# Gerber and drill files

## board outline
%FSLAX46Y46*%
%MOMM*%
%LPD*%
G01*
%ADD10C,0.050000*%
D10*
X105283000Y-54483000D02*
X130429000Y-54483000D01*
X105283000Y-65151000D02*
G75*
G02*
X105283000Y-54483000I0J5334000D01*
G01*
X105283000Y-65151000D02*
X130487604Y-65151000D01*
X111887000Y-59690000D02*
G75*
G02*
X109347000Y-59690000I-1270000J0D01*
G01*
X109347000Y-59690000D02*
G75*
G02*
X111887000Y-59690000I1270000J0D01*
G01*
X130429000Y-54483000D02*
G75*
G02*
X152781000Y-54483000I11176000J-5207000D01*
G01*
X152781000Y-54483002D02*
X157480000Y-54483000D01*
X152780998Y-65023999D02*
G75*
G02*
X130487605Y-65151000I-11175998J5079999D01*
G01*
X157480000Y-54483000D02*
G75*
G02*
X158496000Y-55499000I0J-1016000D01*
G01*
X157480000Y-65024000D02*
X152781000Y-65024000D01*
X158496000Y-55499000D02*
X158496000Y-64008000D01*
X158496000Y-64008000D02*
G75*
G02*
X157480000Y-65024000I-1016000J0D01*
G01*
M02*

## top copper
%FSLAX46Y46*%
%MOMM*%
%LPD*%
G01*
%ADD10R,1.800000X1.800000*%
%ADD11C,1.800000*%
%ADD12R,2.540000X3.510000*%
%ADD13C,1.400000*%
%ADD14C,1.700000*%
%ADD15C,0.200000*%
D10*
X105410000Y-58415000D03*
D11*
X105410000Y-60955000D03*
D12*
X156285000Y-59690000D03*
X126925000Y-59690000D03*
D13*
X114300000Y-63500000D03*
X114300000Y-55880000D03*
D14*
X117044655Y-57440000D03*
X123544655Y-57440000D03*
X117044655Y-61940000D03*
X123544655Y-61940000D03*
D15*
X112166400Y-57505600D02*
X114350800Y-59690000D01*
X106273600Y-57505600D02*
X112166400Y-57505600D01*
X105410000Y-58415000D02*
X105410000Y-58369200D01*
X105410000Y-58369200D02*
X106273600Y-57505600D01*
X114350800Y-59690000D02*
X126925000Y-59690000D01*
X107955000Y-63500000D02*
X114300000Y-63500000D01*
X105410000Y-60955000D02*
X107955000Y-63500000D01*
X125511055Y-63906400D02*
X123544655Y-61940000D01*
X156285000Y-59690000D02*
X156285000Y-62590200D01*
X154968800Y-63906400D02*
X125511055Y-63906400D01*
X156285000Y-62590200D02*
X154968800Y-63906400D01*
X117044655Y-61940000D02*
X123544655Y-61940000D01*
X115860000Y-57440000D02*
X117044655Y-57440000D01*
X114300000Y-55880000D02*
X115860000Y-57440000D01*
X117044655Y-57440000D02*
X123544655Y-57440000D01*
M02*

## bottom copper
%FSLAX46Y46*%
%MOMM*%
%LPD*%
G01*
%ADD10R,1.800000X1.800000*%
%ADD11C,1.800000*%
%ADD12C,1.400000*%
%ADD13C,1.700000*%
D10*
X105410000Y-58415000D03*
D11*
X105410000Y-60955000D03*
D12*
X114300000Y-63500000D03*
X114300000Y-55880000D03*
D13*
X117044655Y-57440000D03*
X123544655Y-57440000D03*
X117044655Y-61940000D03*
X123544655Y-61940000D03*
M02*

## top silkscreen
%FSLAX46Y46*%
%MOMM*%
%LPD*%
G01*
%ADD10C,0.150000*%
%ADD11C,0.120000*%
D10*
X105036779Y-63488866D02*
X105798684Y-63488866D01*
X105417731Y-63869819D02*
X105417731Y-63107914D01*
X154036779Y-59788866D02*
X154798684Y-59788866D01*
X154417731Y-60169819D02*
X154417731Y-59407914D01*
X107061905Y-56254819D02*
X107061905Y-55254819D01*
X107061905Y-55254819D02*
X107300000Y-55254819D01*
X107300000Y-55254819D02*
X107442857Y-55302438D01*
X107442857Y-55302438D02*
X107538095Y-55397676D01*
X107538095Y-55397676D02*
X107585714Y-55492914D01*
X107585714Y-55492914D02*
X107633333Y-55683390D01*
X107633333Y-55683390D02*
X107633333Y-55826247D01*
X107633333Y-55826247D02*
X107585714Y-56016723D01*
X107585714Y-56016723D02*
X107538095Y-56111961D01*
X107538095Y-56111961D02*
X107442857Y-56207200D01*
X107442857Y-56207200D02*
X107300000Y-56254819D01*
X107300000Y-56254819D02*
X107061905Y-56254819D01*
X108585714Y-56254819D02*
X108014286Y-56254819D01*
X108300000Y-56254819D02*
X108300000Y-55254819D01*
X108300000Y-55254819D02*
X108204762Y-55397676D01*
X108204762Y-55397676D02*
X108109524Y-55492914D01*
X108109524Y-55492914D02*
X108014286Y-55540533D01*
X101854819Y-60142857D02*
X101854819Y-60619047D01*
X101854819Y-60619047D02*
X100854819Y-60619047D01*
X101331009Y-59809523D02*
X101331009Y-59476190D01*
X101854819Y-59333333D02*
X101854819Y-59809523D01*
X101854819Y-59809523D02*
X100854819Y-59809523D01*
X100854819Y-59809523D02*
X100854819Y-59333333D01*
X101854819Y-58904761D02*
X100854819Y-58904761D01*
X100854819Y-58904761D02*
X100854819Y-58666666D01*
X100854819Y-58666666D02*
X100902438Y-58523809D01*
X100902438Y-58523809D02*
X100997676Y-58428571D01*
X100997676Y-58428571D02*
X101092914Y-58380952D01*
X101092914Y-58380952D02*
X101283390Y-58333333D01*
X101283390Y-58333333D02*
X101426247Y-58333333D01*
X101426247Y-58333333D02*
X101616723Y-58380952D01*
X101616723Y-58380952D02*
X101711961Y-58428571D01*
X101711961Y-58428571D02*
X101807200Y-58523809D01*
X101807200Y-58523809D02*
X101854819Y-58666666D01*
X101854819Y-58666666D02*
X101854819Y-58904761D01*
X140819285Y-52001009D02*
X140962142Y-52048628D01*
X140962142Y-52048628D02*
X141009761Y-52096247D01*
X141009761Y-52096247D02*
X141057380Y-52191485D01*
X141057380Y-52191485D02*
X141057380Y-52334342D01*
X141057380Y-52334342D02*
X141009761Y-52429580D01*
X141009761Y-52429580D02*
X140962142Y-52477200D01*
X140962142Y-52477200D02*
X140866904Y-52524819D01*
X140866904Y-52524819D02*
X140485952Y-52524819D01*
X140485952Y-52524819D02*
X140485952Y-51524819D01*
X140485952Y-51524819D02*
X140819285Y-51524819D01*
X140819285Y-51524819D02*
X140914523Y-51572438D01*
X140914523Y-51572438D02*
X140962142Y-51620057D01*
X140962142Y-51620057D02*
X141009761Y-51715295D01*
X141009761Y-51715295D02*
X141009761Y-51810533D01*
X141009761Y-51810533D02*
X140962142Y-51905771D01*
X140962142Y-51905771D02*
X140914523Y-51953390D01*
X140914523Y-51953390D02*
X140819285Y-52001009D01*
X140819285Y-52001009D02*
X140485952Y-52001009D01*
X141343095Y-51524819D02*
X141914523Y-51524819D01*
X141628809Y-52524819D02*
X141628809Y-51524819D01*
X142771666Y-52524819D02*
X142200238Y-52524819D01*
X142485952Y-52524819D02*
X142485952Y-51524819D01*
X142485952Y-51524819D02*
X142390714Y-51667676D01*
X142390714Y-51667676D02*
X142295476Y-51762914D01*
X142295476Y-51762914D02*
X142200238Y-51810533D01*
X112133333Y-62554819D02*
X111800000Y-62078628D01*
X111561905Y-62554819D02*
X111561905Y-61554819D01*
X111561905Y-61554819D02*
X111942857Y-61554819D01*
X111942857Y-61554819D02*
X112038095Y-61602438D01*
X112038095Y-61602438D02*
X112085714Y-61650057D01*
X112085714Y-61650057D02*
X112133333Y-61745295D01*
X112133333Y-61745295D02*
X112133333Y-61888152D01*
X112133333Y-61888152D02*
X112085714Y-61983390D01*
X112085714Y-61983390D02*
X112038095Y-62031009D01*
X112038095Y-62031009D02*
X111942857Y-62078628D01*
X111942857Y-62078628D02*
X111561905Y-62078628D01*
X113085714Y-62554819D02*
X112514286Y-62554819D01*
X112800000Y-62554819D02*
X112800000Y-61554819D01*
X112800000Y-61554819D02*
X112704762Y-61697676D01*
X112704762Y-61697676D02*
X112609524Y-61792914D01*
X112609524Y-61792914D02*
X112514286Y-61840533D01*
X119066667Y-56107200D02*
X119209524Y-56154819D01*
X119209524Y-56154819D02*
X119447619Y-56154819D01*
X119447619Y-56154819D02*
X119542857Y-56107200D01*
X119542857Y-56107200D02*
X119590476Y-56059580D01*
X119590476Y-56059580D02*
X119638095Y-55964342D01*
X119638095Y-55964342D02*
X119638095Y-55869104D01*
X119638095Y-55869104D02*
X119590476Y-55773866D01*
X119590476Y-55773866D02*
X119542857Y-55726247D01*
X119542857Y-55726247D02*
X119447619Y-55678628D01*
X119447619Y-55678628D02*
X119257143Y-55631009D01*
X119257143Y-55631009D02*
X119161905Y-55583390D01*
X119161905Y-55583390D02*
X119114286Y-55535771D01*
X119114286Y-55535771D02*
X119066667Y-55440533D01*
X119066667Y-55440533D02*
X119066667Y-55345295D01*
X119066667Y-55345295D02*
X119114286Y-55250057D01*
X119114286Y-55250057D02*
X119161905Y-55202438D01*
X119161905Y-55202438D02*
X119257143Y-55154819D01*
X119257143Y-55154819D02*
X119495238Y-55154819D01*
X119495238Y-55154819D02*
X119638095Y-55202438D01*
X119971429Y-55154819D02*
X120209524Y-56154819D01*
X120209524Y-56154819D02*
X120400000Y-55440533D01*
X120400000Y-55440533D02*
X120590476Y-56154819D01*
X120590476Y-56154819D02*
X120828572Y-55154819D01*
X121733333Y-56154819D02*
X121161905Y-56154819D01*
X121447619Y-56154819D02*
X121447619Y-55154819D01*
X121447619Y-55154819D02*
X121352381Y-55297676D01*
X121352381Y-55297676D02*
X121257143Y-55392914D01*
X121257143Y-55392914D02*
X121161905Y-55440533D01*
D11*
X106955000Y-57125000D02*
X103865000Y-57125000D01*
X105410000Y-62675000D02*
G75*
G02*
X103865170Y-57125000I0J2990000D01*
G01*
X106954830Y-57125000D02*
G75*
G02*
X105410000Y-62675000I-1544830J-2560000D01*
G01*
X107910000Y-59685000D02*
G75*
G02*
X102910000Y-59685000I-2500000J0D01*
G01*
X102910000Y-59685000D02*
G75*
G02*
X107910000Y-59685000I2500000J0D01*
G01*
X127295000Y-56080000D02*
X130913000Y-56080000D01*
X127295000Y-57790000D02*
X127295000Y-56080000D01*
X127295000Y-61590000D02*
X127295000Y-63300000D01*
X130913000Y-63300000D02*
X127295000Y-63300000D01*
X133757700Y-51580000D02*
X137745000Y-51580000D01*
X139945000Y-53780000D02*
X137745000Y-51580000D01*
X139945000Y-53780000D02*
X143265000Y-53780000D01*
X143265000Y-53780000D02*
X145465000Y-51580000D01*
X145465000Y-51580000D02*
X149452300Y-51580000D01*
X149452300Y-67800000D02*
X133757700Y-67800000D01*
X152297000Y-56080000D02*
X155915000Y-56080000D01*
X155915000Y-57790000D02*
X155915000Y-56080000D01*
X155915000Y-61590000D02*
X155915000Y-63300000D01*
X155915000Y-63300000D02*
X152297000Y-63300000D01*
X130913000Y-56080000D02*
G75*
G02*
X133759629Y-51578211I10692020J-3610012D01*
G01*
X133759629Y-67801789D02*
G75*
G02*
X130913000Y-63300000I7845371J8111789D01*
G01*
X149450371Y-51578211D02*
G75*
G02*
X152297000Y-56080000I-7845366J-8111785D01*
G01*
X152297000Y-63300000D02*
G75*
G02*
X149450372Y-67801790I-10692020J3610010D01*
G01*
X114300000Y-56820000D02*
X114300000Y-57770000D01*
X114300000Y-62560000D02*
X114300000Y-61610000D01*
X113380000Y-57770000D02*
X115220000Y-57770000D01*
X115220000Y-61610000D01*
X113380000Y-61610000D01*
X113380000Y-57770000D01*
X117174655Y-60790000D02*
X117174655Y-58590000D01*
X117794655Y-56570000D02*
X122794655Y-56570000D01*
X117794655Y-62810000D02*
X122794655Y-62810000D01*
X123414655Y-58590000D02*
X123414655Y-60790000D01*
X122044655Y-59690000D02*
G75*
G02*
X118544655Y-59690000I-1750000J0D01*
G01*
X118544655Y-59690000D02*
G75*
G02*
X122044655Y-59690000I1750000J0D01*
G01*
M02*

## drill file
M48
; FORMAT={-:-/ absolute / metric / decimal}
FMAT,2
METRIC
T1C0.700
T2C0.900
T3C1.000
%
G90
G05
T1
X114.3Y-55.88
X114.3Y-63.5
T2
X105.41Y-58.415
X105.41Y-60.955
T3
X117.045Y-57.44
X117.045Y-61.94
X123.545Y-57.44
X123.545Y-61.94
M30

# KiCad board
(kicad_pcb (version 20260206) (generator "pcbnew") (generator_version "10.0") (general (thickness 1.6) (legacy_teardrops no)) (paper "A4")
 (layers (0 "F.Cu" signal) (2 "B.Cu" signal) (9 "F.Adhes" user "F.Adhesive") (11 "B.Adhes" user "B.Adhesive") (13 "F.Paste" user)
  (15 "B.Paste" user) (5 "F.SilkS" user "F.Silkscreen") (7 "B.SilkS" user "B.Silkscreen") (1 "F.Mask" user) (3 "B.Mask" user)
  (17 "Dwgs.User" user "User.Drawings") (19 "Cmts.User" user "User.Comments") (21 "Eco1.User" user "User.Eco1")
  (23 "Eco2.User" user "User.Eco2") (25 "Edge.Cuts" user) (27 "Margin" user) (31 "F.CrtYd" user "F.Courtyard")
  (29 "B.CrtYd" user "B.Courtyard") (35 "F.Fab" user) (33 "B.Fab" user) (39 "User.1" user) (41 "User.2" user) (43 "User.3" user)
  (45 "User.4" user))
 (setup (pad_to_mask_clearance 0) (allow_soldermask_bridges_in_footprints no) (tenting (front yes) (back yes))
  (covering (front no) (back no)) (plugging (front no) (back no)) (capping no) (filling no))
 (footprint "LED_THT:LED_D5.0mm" (layer "F.Cu") (at 105.41 58.415 -90)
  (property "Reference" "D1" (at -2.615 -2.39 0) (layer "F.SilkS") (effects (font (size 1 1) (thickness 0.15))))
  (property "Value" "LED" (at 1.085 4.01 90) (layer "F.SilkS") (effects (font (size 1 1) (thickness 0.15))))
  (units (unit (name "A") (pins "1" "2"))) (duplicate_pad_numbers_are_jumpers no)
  (fp_line (start -1.29 -1.545) (end -1.29 1.545) (stroke (width 0.12) (type solid)) (layer "F.SilkS"))
  (fp_arc (start 4.26 0) (mid 2.071779 2.880495) (end -1.29 1.54483) (stroke (width 0.12) (type solid)) (layer "F.SilkS"))
  (fp_arc (start -1.29 -1.54483) (mid 2.071779 -2.880495) (end 4.26 0) (stroke (width 0.12) (type solid)) (layer "F.SilkS"))
  (fp_circle (center 1.27 0) (end 3.77 0) (stroke (width 0.12) (type solid)) (fill no) (layer "F.SilkS"))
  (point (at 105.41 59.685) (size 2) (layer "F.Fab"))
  (pad "1" thru_hole rect (at 0 0 270) (size 1.8 1.8) (drill 0.9) (layers "*.Cu" "*.Mask") (remove_unused_layers no) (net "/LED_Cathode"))
  (pad "2" thru_hole circle (at 2.54 0 270) (size 1.8 1.8) (drill 0.9) (layers "*.Cu" "*.Mask") (remove_unused_layers no) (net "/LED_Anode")))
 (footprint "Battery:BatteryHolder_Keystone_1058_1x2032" (layer "F.Cu") (at 141.605 59.69 180)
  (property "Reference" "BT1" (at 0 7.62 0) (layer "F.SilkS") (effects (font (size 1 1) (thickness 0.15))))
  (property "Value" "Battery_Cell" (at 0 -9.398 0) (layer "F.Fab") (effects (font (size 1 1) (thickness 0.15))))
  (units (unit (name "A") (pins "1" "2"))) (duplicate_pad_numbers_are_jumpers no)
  (fp_line (start 14.31 3.61) (end 10.692 3.61) (stroke (width 0.12) (type solid)) (layer "F.SilkS"))
  (fp_line (start 14.31 1.9) (end 14.31 3.61) (stroke (width 0.12) (type solid)) (layer "F.SilkS"))
  (fp_line (start 14.31 -1.9) (end 14.31 -3.61) (stroke (width 0.12) (type solid)) (layer "F.SilkS"))
  (fp_line (start 10.692 -3.61) (end 14.31 -3.61) (stroke (width 0.12) (type solid)) (layer "F.SilkS"))
  (fp_line (start 7.8473 8.11) (end 3.86 8.11) (stroke (width 0.12) (type solid)) (layer "F.SilkS"))
  (fp_line (start 1.66 5.91) (end 3.86 8.11) (stroke (width 0.12) (type solid)) (layer "F.SilkS"))
  (fp_line (start 1.66 5.91) (end -1.66 5.91) (stroke (width 0.12) (type solid)) (layer "F.SilkS"))
  (fp_line (start -1.66 5.91) (end -3.86 8.11) (stroke (width 0.12) (type solid)) (layer "F.SilkS"))
  (fp_line (start -3.86 8.11) (end -7.8473 8.11) (stroke (width 0.12) (type solid)) (layer "F.SilkS"))
  (fp_line (start -7.8473 -8.11) (end 7.8473 -8.11) (stroke (width 0.12) (type solid)) (layer "F.SilkS"))
  (fp_line (start -10.692 3.61) (end -14.31 3.61) (stroke (width 0.12) (type solid)) (layer "F.SilkS"))
  (fp_line (start -14.31 1.9) (end -14.31 3.61) (stroke (width 0.12) (type solid)) (layer "F.SilkS"))
  (fp_line (start -14.31 -1.9) (end -14.31 -3.61) (stroke (width 0.12) (type solid)) (layer "F.SilkS"))
  (fp_line (start -14.31 -3.61) (end -10.692 -3.61) (stroke (width 0.12) (type solid)) (layer "F.SilkS"))
  (fp_arc (start 10.692 3.61) (mid 9.538084 6.031244) (end 7.845371 8.111789) (stroke (width 0.12) (type solid)) (layer "F.SilkS"))
  (fp_arc (start 7.845371 -8.111789) (mid 9.538085 -6.031244) (end 10.692 -3.61) (stroke (width 0.12) (type solid)) (layer "F.SilkS"))
  (fp_arc (start -7.845371 8.111789) (mid -9.538085 6.031244) (end -10.692 3.61) (stroke (width 0.12) (type solid)) (layer "F.SilkS"))
  (fp_arc (start -10.692 -3.61) (mid -9.538084 -6.031244) (end -7.845371 -8.111789) (stroke (width 0.12) (type solid)) (layer "F.SilkS"))
  (pad "1" smd rect (at -14.68 0 180) (size 2.54 3.51) (layers "F.Cu" "F.Mask" "F.Paste") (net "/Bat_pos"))
  (pad "2" smd rect (at 14.68 0 180) (size 2.54 3.51) (layers "F.Cu" "F.Mask" "F.Paste") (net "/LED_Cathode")))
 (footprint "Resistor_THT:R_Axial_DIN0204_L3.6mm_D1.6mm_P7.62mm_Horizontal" (layer "F.Cu") (at 114.3 63.5 90)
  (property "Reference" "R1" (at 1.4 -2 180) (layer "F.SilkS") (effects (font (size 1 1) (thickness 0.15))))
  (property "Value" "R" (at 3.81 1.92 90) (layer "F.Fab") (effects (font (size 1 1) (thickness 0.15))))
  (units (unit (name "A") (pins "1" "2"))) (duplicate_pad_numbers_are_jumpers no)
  (fp_line (start 6.68 0) (end 5.73 0) (stroke (width 0.12) (type solid)) (layer "F.SilkS"))
  (fp_line (start 0.94 0) (end 1.89 0) (stroke (width 0.12) (type solid)) (layer "F.SilkS"))
  (fp_rect (start 1.89 -0.92) (end 5.73 0.92) (stroke (width 0.12) (type solid)) (fill no) (layer "F.SilkS"))
  (pad "1" thru_hole circle (at 0 0 90) (size 1.4 1.4) (drill 0.7) (layers "*.Cu" "*.Mask") (remove_unused_layers no) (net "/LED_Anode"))
  (pad "2" thru_hole circle (at 7.62 0 90) (size 1.4 1.4) (drill 0.7) (layers "*.Cu" "*.Mask") (remove_unused_layers no)
   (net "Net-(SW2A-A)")))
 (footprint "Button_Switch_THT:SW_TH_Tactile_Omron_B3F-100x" (layer "F.Cu") (at 117.044655 57.44)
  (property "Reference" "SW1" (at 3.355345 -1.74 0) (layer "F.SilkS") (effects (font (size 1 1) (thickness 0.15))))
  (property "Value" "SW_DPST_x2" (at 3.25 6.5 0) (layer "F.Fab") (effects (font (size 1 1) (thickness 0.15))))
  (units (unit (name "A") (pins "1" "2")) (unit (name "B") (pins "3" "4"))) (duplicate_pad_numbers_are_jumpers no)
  (fp_line (start 0.13 3.35) (end 0.13 1.15) (stroke (width 0.12) (type solid)) (layer "F.SilkS"))
  (fp_line (start 0.75 -0.87) (end 5.75 -0.87) (stroke (width 0.12) (type solid)) (layer "F.SilkS"))
  (fp_line (start 0.75 5.37) (end 5.75 5.37) (stroke (width 0.12) (type solid)) (layer "F.SilkS"))
  (fp_line (start 6.37 1.15) (end 6.37 3.35) (stroke (width 0.12) (type solid)) (layer "F.SilkS"))
  (fp_circle (center 3.25 2.25) (end 5 2.25) (stroke (width 0.12) (type solid)) (fill no) (layer "F.SilkS"))
  (pad "1" thru_hole circle (at 0 0) (size 1.7 1.7) (drill 1) (layers "*.Cu" "*.Mask") (remove_unused_layers no) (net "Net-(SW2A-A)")
   (thermal_bridge_angle 90))
  (pad "1" thru_hole circle (at 6.5 0) (size 1.7 1.7) (drill 1) (layers "*.Cu" "*.Mask") (remove_unused_layers no) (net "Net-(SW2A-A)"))
  (pad "2" thru_hole circle (at 0 4.5) (size 1.7 1.7) (drill 1) (layers "*.Cu" "*.Mask") (remove_unused_layers no) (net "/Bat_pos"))
  (pad "2" thru_hole circle (at 6.5 4.5) (size 1.7 1.7) (drill 1) (layers "*.Cu" "*.Mask") (remove_unused_layers no) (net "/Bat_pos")))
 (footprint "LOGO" (layer "B.Cu") (at 141.605 59.69 180)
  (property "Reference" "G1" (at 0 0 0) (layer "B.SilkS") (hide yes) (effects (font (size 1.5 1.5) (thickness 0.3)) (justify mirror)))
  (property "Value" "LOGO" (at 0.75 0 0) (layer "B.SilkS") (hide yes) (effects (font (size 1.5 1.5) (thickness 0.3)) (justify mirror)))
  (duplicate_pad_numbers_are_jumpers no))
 (gr_line (start 105.283 54.483) (end 130.429 54.483) (stroke (width 0.05) (type default)) (locked yes) (layer "Edge.Cuts"))
 (gr_arc (start 105.283 65.151) (mid 99.949 59.817) (end 105.283 54.483) (stroke (width 0.05) (type default)) (locked yes)
  (layer "Edge.Cuts"))
 (gr_line (start 105.283 65.151) (end 130.487604 65.151) (stroke (width 0.05) (type default)) (locked yes) (layer "Edge.Cuts"))
 (gr_circle (center 110.617 59.69) (end 111.887 59.69) (stroke (width 0.05) (type default)) (fill no) (layer "Edge.Cuts"))
 (gr_arc (start 130.429 54.483) (mid 141.605 47.36053) (end 152.781 54.483) (stroke (width 0.05) (type default)) (locked yes)
  (layer "Edge.Cuts"))
 (gr_line (start 152.781 54.483002) (end 157.48 54.483) (stroke (width 0.05) (type default)) (locked yes) (layer "Edge.Cuts"))
 (gr_arc (start 152.780998 65.023999) (mid 141.674935 72.220173) (end 130.487604 65.151) (stroke (width 0.05) (type default)) (locked yes)
  (layer "Edge.Cuts"))
 (gr_arc (start 157.48 54.483) (mid 158.19842 54.78058) (end 158.496 55.499) (stroke (width 0.05) (type default)) (locked yes)
  (layer "Edge.Cuts"))
 (gr_line (start 157.48 65.024) (end 152.781 65.024) (stroke (width 0.05) (type default)) (locked yes) (layer "Edge.Cuts"))
 (gr_line (start 158.496 55.499) (end 158.496 64.008) (stroke (width 0.05) (type default)) (locked yes) (layer "Edge.Cuts"))
 (gr_arc (start 158.496 64.008) (mid 158.19842 64.72642) (end 157.48 65.024) (stroke (width 0.05) (type default)) (locked yes)
  (layer "Edge.Cuts"))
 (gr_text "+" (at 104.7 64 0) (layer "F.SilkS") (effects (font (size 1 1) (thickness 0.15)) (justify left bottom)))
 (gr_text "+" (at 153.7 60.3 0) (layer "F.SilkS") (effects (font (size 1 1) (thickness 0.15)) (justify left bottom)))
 (segment (start 112.1664 57.5056) (end 114.3508 59.69) (width 0.2) (layer "F.Cu") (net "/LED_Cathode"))
 (segment (start 106.2736 57.5056) (end 112.1664 57.5056) (width 0.2) (layer "F.Cu") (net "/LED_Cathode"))
 (segment (start 105.41 58.415) (end 105.41 58.3692) (width 0.2) (layer "F.Cu") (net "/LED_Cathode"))
 (segment (start 105.41 58.3692) (end 106.2736 57.5056) (width 0.2) (layer "F.Cu") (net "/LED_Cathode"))
 (segment (start 114.3508 59.69) (end 126.925 59.69) (width 0.2) (layer "F.Cu") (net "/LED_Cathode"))
 (segment (start 107.955 63.5) (end 114.3 63.5) (width 0.2) (layer "F.Cu") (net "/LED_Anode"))
 (segment (start 105.41 60.955) (end 107.955 63.5) (width 0.2) (layer "F.Cu") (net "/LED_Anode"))
 (segment (start 125.511055 63.9064) (end 123.544655 61.94) (width 0.2) (layer "F.Cu") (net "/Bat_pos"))
 (segment (start 156.285 59.69) (end 156.285 62.5902) (width 0.2) (layer "F.Cu") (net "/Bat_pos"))
 (segment (start 154.9688 63.9064) (end 125.511055 63.9064) (width 0.2) (layer "F.Cu") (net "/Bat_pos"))
 (segment (start 156.285 62.5902) (end 154.9688 63.9064) (width 0.2) (layer "F.Cu") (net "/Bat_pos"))
 (segment (start 117.044655 61.94) (end 123.544655 61.94) (width 0.2) (layer "F.Cu") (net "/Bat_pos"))
 (segment (start 115.86 57.44) (end 117.044655 57.44) (width 0.2) (layer "F.Cu") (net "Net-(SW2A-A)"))
 (segment (start 114.3 55.88) (end 115.86 57.44) (width 0.2) (layer "F.Cu") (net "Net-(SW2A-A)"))
 (segment (start 117.044655 57.44) (end 123.544655 57.44) (width 0.2) (layer "F.Cu") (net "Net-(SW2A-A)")))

